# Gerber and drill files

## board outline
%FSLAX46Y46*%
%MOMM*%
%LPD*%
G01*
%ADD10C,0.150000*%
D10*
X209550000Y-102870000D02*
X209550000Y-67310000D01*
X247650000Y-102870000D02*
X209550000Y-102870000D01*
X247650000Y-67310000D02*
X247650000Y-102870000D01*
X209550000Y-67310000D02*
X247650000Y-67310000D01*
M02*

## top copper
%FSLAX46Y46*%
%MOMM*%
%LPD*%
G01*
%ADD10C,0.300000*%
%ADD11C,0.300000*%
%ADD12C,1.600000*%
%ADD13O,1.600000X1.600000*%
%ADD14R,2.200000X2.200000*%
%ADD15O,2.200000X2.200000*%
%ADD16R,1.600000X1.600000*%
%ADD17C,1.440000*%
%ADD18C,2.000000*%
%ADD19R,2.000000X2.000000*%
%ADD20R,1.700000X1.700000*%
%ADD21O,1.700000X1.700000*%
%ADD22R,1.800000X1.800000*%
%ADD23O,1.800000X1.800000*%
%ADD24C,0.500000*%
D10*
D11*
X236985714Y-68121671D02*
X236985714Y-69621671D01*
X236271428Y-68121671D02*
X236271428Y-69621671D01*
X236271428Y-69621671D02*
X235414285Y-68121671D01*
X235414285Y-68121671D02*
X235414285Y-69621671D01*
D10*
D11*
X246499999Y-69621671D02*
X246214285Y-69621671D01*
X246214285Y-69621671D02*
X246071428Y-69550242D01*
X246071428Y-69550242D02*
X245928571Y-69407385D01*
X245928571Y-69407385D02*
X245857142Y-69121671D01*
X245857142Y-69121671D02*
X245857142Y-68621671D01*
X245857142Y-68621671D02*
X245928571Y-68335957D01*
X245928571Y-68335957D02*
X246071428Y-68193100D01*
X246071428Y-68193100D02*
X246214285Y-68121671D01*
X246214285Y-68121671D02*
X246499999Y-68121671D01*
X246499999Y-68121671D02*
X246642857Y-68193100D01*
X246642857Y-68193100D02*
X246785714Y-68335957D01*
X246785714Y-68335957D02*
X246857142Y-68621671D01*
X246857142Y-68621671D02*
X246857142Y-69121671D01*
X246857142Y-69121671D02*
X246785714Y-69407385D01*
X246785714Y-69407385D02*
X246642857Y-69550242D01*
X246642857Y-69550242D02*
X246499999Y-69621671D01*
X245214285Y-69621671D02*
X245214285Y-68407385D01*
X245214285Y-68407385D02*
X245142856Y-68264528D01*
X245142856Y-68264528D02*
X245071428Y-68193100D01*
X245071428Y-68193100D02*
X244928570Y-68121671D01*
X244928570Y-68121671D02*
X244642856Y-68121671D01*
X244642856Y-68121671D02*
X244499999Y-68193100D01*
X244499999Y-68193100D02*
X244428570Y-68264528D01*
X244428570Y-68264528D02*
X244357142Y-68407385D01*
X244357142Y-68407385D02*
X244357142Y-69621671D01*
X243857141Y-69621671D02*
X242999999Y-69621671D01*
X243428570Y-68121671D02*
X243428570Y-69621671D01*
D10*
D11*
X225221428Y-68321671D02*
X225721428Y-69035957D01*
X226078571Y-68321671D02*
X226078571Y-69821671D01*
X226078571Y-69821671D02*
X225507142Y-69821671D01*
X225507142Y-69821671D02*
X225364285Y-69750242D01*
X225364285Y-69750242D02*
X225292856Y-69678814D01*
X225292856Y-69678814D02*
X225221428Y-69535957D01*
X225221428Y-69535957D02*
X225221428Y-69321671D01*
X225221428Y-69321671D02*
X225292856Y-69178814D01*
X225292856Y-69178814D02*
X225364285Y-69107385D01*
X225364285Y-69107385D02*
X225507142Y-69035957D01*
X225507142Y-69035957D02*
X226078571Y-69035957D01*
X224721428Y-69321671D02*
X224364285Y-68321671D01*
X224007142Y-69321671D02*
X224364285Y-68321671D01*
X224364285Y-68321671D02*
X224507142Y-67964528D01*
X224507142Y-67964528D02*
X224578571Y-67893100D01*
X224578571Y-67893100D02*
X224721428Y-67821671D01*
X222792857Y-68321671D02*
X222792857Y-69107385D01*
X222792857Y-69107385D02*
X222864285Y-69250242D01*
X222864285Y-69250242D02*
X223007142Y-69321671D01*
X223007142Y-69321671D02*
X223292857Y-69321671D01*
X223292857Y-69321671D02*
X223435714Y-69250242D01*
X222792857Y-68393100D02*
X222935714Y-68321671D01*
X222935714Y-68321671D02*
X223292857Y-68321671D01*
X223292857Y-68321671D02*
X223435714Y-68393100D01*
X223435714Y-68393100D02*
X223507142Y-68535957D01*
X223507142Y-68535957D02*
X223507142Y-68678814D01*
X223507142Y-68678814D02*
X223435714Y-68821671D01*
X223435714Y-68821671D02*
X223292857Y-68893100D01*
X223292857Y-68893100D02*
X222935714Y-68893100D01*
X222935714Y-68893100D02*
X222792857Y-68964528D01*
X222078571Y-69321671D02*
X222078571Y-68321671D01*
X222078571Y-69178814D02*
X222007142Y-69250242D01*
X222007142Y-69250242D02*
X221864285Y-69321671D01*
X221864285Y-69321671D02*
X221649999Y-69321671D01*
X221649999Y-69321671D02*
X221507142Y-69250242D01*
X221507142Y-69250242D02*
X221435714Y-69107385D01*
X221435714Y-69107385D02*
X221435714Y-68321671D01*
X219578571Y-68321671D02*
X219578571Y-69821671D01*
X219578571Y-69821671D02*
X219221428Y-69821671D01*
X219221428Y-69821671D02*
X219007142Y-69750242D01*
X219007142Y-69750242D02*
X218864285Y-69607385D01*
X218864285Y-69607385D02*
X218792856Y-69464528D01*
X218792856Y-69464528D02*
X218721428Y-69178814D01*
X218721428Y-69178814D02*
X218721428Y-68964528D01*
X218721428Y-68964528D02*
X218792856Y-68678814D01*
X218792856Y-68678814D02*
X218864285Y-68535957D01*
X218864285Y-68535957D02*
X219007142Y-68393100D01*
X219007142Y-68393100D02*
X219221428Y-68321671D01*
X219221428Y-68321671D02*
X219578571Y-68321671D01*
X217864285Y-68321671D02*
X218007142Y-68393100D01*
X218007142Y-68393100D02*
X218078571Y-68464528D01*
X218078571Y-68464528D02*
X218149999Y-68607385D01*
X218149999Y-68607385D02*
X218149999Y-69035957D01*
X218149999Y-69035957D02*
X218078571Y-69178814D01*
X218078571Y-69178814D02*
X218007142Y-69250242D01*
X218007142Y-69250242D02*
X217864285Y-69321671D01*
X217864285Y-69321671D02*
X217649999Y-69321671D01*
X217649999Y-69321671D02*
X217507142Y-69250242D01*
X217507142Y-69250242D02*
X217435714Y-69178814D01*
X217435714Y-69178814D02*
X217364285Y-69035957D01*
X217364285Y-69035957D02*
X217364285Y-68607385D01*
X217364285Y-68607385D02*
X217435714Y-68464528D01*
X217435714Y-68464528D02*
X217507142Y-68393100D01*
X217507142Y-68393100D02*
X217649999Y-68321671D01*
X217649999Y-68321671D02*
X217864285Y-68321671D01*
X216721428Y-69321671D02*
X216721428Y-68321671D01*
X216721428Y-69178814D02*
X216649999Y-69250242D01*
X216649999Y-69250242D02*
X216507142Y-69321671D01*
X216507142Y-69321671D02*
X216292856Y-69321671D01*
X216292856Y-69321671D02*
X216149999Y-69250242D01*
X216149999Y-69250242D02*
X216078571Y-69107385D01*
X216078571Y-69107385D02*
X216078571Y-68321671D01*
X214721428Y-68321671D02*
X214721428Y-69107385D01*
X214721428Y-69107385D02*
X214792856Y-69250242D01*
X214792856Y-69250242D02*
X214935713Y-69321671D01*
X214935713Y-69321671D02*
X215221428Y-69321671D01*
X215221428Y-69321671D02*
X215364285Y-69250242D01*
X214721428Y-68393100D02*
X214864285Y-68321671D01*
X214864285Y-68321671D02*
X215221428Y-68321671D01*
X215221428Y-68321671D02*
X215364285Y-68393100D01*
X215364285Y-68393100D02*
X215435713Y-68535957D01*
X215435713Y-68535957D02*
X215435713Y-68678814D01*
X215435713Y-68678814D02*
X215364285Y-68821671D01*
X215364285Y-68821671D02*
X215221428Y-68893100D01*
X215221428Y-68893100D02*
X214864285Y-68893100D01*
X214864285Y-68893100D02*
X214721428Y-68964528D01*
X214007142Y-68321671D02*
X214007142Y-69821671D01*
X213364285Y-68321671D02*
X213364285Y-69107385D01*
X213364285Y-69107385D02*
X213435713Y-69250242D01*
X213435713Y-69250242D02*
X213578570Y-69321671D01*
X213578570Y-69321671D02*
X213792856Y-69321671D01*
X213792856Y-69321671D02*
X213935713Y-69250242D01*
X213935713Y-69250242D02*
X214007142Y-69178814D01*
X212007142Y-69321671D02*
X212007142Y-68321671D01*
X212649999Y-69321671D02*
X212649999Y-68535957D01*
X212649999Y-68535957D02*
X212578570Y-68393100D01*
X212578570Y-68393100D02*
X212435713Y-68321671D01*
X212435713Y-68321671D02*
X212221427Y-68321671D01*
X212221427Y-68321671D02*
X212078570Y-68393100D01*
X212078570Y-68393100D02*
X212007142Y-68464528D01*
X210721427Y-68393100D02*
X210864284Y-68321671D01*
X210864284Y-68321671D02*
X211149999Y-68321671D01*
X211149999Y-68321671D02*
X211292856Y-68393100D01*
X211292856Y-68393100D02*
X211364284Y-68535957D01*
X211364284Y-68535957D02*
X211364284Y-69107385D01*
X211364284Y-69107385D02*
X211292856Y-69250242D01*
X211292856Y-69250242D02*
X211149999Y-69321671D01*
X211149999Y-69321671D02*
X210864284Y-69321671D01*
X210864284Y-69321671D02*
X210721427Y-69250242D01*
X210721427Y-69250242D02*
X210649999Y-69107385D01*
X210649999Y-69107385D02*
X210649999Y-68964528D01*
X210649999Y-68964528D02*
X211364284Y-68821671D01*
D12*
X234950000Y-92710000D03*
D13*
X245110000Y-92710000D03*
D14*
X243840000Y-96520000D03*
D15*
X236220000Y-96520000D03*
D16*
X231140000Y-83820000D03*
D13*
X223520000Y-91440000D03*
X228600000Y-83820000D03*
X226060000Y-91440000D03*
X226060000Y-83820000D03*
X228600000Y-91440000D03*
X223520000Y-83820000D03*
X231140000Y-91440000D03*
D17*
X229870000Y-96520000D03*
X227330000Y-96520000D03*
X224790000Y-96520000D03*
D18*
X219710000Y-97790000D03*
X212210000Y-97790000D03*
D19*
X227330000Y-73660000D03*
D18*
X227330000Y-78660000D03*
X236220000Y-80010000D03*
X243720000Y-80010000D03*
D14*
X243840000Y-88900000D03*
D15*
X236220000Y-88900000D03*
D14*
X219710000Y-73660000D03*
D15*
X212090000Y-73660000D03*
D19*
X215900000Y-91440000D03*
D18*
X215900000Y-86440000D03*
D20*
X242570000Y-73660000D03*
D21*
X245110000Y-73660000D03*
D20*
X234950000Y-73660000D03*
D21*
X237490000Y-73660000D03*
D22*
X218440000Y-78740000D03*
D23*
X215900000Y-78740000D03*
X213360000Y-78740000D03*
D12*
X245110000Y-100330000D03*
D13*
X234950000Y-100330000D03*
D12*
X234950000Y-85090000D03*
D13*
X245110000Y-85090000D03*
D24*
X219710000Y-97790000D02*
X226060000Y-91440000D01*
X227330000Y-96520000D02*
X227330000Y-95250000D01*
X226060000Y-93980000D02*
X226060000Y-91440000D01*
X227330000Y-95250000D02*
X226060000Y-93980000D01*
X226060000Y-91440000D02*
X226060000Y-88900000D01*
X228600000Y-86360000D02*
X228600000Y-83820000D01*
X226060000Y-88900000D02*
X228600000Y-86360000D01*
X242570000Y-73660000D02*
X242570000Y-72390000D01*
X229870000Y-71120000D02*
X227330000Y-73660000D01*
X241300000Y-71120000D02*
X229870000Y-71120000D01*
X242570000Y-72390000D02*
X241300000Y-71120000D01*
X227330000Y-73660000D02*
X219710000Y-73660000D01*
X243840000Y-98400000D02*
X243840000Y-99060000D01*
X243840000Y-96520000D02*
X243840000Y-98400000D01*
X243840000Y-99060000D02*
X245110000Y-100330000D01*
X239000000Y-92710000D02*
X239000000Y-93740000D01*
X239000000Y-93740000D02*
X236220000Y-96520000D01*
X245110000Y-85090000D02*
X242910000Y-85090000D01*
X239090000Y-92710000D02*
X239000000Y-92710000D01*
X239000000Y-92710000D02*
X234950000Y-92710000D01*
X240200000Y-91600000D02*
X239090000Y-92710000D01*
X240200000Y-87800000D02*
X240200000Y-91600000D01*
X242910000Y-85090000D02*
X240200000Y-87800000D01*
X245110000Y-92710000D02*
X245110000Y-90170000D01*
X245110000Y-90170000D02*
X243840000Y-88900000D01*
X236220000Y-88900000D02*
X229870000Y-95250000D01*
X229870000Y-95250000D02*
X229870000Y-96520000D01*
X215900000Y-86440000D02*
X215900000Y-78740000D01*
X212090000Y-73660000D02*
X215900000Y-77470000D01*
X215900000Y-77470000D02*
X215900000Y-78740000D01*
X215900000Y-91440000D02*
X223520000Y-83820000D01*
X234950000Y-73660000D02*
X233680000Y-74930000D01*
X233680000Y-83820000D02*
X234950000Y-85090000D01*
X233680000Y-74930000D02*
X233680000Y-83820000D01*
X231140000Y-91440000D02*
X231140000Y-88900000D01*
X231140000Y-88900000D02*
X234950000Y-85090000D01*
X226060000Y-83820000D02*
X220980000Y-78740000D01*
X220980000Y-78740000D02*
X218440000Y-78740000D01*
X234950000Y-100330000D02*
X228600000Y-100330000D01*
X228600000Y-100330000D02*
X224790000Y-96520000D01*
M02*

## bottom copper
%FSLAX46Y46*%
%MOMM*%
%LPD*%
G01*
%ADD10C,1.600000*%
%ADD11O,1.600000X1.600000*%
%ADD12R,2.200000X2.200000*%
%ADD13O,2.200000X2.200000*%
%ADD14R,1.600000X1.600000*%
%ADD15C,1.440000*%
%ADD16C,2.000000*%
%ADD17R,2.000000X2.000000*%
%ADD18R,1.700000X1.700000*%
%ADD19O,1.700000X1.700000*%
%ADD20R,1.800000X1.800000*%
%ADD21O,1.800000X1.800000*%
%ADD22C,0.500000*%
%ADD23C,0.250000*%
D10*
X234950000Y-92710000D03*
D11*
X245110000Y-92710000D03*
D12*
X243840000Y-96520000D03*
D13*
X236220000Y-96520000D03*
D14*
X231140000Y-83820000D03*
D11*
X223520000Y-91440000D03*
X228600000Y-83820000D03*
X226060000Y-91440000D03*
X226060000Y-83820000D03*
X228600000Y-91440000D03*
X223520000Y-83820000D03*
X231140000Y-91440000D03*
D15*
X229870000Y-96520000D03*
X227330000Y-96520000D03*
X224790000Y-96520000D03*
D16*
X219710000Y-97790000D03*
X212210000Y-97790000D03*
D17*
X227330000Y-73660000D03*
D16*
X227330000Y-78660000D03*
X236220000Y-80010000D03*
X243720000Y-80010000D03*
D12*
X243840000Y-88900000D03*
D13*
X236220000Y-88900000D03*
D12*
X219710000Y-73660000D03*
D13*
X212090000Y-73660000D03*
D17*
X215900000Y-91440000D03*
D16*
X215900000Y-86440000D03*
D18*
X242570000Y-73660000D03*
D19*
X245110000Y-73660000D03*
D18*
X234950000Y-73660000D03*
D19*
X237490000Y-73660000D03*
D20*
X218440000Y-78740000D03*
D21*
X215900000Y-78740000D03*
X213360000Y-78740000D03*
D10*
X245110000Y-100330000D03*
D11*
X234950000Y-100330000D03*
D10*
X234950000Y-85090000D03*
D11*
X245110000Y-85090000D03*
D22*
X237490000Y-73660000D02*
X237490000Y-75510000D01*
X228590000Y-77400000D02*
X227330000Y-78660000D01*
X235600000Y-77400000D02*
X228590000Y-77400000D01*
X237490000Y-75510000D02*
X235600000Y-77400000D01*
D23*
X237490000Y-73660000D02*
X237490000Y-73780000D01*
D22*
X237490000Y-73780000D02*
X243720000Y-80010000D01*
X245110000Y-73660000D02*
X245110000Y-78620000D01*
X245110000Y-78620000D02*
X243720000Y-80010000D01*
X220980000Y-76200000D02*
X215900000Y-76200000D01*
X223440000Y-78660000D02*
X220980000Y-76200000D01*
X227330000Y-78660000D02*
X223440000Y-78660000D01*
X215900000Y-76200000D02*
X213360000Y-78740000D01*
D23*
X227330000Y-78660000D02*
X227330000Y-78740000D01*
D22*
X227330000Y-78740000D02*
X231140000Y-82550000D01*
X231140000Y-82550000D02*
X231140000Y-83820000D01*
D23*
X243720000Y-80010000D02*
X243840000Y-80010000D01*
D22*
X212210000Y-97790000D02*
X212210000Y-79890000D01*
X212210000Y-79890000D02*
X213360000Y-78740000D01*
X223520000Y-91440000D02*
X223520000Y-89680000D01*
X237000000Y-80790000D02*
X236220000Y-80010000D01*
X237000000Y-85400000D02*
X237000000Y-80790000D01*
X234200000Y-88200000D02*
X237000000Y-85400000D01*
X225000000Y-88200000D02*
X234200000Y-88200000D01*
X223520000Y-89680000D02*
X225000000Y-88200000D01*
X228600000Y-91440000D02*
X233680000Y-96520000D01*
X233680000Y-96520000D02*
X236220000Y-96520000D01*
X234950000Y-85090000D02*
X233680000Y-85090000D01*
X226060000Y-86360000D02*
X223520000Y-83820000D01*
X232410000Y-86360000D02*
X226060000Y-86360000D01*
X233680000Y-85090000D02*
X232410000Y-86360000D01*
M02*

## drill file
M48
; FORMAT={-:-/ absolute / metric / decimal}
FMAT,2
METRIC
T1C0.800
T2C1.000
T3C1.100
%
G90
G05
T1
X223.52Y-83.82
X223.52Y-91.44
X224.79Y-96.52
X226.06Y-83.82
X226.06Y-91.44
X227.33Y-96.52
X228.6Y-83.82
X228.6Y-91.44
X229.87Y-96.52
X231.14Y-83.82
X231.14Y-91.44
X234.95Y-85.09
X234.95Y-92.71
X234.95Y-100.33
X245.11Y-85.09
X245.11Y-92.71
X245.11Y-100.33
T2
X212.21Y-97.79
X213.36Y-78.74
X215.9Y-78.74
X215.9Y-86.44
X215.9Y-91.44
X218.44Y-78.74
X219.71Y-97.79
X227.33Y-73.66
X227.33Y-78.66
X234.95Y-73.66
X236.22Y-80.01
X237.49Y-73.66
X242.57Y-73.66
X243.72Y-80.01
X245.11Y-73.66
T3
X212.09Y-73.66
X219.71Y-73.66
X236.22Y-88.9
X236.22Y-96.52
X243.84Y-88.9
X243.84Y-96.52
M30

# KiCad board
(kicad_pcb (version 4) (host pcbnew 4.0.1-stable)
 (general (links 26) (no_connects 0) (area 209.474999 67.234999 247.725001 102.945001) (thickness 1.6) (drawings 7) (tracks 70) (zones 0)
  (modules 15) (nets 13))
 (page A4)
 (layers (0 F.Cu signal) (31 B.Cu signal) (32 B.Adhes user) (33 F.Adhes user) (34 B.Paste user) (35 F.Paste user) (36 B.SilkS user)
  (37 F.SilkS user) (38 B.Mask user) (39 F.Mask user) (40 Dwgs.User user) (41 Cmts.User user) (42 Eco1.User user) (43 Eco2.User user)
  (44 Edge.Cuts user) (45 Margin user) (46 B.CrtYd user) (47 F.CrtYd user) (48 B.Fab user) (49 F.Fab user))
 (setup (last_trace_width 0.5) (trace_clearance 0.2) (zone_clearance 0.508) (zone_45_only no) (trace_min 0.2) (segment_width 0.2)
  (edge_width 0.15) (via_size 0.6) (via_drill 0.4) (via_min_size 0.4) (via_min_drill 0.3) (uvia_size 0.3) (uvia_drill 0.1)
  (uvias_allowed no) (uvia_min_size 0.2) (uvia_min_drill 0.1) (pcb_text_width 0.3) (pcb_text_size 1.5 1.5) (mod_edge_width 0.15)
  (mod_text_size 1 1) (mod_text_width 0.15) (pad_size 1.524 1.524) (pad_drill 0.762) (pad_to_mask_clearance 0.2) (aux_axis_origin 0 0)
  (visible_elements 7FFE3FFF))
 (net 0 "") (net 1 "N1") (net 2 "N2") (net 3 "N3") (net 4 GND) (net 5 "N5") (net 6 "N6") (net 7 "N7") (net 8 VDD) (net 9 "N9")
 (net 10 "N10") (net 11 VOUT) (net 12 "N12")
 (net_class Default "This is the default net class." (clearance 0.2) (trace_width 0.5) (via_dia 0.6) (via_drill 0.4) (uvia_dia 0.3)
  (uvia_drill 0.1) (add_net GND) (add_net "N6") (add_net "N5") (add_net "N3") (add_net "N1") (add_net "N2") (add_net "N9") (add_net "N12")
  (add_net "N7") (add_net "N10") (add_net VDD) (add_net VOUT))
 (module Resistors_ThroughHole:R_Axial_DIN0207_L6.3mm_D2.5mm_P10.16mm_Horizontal (layer F.Cu) (at 234.95 92.71)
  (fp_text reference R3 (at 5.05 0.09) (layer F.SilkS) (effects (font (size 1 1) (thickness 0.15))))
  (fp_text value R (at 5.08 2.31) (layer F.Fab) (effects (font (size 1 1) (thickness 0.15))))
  (pad 1 thru_hole circle (at 0 0) (size 1.6 1.6) (drill 0.8) (layers *.Cu *.Mask) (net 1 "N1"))
  (pad 2 thru_hole oval (at 10.16 0) (size 1.6 1.6) (drill 0.8) (layers *.Cu *.Mask) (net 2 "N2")))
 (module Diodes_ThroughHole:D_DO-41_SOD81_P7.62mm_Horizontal (layer F.Cu) (at 243.84 96.52 180)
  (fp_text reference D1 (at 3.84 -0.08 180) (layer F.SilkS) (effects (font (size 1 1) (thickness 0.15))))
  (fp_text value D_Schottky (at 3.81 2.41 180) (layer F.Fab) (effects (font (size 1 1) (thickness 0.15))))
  (pad 1 thru_hole rect (at 0 0 180) (size 2.2 2.2) (drill 1.1) (layers *.Cu *.Mask) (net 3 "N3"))
  (pad 2 thru_hole oval (at 7.62 0 180) (size 2.2 2.2) (drill 1.1) (layers *.Cu *.Mask) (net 1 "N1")))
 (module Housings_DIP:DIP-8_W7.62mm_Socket (layer F.Cu) (at 231.14 83.82 270)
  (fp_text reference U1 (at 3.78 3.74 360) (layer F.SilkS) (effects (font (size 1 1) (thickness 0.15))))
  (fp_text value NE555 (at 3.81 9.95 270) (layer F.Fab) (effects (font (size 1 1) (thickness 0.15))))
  (pad 1 thru_hole rect (at 0 0 270) (size 1.6 1.6) (drill 0.8) (layers *.Cu *.Mask) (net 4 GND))
  (pad 5 thru_hole oval (at 7.62 7.62 270) (size 1.6 1.6) (drill 0.8) (layers *.Cu *.Mask) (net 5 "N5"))
  (pad 2 thru_hole oval (at 0 2.54 270) (size 1.6 1.6) (drill 0.8) (layers *.Cu *.Mask) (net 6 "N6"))
  (pad 6 thru_hole oval (at 7.62 5.08 270) (size 1.6 1.6) (drill 0.8) (layers *.Cu *.Mask) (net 6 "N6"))
  (pad 3 thru_hole oval (at 0 5.08 270) (size 1.6 1.6) (drill 0.8) (layers *.Cu *.Mask) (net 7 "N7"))
  (pad 7 thru_hole oval (at 7.62 2.54 270) (size 1.6 1.6) (drill 0.8) (layers *.Cu *.Mask) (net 1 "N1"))
  (pad 4 thru_hole oval (at 0 7.62 270) (size 1.6 1.6) (drill 0.8) (layers *.Cu *.Mask) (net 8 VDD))
  (pad 8 thru_hole oval (at 7.62 0 270) (size 1.6 1.6) (drill 0.8) (layers *.Cu *.Mask) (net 8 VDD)))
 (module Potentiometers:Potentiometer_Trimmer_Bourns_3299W (layer F.Cu) (at 229.87 96.52)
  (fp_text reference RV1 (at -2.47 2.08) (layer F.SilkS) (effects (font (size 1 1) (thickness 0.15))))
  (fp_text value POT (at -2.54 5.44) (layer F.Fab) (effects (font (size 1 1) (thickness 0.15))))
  (pad 1 thru_hole circle (at 0 0) (size 1.44 1.44) (drill 0.8) (layers *.Cu *.Mask) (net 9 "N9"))
  (pad 2 thru_hole circle (at -2.54 0) (size 1.44 1.44) (drill 0.8) (layers *.Cu *.Mask) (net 6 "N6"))
  (pad 3 thru_hole circle (at -5.08 0) (size 1.44 1.44) (drill 0.8) (layers *.Cu *.Mask) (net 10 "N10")))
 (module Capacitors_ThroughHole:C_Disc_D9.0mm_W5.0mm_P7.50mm (layer F.Cu) (at 219.71 97.79 180)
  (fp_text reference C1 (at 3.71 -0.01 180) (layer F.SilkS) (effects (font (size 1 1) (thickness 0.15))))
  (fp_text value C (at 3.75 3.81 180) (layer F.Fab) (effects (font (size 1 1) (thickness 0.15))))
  (pad 1 thru_hole circle (at 0 0 180) (size 2 2) (drill 1) (layers *.Cu *.Mask) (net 6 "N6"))
  (pad 2 thru_hole circle (at 7.5 0 180) (size 2 2) (drill 1) (layers *.Cu *.Mask) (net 4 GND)))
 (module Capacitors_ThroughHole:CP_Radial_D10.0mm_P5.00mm (layer F.Cu) (at 227.33 73.66 270)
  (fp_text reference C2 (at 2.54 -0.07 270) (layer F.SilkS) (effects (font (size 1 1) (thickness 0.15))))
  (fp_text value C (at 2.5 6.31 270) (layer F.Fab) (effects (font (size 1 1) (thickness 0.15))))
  (pad 1 thru_hole rect (at 0 0 270) (size 2 2) (drill 1) (layers *.Cu *.Mask) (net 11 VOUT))
  (pad 2 thru_hole circle (at 5 0 270) (size 2 2) (drill 1) (layers *.Cu *.Mask) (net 4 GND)))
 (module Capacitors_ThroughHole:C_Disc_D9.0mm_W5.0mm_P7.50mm (layer F.Cu) (at 236.22 80.01)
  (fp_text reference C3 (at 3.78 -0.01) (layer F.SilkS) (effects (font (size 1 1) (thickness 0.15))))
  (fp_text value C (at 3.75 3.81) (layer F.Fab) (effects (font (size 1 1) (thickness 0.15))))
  (pad 1 thru_hole circle (at 0 0) (size 2 2) (drill 1) (layers *.Cu *.Mask) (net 5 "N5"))
  (pad 2 thru_hole circle (at 7.5 0) (size 2 2) (drill 1) (layers *.Cu *.Mask) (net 4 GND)))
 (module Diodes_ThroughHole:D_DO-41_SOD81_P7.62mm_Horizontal (layer F.Cu) (at 243.84 88.9 180)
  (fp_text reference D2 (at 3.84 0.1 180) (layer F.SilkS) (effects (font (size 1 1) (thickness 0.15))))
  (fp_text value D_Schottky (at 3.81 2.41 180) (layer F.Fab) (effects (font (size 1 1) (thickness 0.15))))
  (pad 1 thru_hole rect (at 0 0 180) (size 2.2 2.2) (drill 1.1) (layers *.Cu *.Mask) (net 2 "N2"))
  (pad 2 thru_hole oval (at 7.62 0 180) (size 2.2 2.2) (drill 1.1) (layers *.Cu *.Mask) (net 9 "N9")))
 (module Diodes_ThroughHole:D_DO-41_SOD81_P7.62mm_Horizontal (layer F.Cu) (at 219.71 73.66 180)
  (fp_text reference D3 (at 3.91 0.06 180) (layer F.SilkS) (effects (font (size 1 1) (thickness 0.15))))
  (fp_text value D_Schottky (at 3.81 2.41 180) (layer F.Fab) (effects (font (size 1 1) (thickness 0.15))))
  (pad 1 thru_hole rect (at 0 0 180) (size 2.2 2.2) (drill 1.1) (layers *.Cu *.Mask) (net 11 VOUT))
  (pad 2 thru_hole oval (at 7.62 0 180) (size 2.2 2.2) (drill 1.1) (layers *.Cu *.Mask) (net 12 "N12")))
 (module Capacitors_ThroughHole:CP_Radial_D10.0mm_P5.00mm (layer F.Cu) (at 215.9 91.44 90)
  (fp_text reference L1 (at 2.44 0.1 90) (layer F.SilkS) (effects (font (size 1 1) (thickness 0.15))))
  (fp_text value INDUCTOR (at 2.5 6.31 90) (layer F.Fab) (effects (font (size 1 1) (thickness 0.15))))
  (pad 1 thru_hole rect (at 0 0 90) (size 2 2) (drill 1) (layers *.Cu *.Mask) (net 8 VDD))
  (pad 2 thru_hole circle (at 5 0 90) (size 2 2) (drill 1) (layers *.Cu *.Mask) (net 12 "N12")))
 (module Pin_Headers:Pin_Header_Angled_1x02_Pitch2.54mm (layer F.Cu) (at 242.57 73.66 90)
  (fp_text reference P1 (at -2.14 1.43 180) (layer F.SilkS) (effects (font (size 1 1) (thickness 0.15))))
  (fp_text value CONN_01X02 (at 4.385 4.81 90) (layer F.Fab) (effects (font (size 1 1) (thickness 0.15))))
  (pad 1 thru_hole rect (at 0 0 90) (size 1.7 1.7) (drill 1) (layers *.Cu *.Mask) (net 11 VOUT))
  (pad 2 thru_hole oval (at 0 2.54 90) (size 1.7 1.7) (drill 1) (layers *.Cu *.Mask) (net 4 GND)))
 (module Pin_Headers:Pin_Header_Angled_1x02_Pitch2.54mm (layer F.Cu) (at 234.95 73.66 90)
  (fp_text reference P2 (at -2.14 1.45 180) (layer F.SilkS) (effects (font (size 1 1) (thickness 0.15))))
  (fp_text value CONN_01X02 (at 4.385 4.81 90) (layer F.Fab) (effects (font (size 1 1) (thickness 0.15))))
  (pad 1 thru_hole rect (at 0 0 90) (size 1.7 1.7) (drill 1) (layers *.Cu *.Mask) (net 8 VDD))
  (pad 2 thru_hole oval (at 0 2.54 90) (size 1.7 1.7) (drill 1) (layers *.Cu *.Mask) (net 4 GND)))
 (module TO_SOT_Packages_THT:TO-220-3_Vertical (layer F.Cu) (at 218.44 78.74 180)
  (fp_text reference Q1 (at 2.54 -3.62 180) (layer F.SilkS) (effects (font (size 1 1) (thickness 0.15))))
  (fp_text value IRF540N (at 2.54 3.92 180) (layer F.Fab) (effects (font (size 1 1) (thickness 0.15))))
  (pad 1 thru_hole rect (at 0 0 180) (size 1.8 1.8) (drill 1) (layers *.Cu *.Mask) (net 7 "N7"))
  (pad 2 thru_hole oval (at 2.54 0 180) (size 1.8 1.8) (drill 1) (layers *.Cu *.Mask) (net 12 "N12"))
  (pad 3 thru_hole oval (at 5.08 0 180) (size 1.8 1.8) (drill 1) (layers *.Cu *.Mask) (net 4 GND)))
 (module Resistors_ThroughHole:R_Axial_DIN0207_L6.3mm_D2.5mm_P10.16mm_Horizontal (layer F.Cu) (at 245.11 100.33 180)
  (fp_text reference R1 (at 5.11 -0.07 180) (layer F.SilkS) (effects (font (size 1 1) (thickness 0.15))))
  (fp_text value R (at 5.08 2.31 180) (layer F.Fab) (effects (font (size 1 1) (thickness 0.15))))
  (pad 1 thru_hole circle (at 0 0 180) (size 1.6 1.6) (drill 0.8) (layers *.Cu *.Mask) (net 3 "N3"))
  (pad 2 thru_hole oval (at 10.16 0 180) (size 1.6 1.6) (drill 0.8) (layers *.Cu *.Mask) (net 10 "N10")))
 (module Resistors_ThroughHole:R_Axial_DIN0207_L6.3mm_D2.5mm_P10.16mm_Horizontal (layer F.Cu) (at 234.95 85.09)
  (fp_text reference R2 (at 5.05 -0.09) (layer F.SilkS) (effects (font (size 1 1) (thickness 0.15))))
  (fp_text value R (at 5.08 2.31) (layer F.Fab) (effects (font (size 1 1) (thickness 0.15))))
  (pad 1 thru_hole circle (at 0 0) (size 1.6 1.6) (drill 0.8) (layers *.Cu *.Mask) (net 8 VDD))
  (pad 2 thru_hole oval (at 10.16 0) (size 1.6 1.6) (drill 0.8) (layers *.Cu *.Mask) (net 1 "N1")))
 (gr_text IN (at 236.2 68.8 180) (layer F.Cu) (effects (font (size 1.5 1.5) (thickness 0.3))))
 (gr_line (start 209.55 102.87) (end 209.55 67.31) (angle 90) (layer Edge.Cuts) (width 0.15))
 (gr_line (start 247.65 102.87) (end 209.55 102.87) (angle 90) (layer Edge.Cuts) (width 0.15))
 (gr_line (start 247.65 67.31) (end 247.65 102.87) (angle 90) (layer Edge.Cuts) (width 0.15))
 (gr_line (start 209.55 67.31) (end 247.65 67.31) (angle 90) (layer Edge.Cuts) (width 0.15))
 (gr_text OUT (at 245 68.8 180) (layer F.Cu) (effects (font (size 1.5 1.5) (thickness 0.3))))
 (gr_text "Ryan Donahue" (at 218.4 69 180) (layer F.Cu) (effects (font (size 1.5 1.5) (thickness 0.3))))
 (segment (start 219.71 97.79) (end 226.06 91.44) (width 0.5) (layer F.Cu) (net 6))
 (segment (start 227.33 96.52) (end 227.33 95.25) (width 0.5) (layer F.Cu) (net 6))
 (segment (start 226.06 93.98) (end 226.06 91.44) (width 0.5) (layer F.Cu) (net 6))
 (segment (start 227.33 95.25) (end 226.06 93.98) (width 0.5) (layer F.Cu) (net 6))
 (segment (start 226.06 91.44) (end 226.06 88.9) (width 0.5) (layer F.Cu) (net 6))
 (segment (start 228.6 86.36) (end 228.6 83.82) (width 0.5) (layer F.Cu) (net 6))
 (segment (start 226.06 88.9) (end 228.6 86.36) (width 0.5) (layer F.Cu) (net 6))
 (segment (start 237.49 73.66) (end 237.49 75.51) (width 0.5) (layer B.Cu) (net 4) (status 400000))
 (segment (start 228.59 77.4) (end 227.33 78.66) (width 0.5) (layer B.Cu) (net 4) (status 800000))
 (segment (start 235.6 77.4) (end 228.59 77.4) (width 0.5) (layer B.Cu) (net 4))
 (segment (start 237.49 75.51) (end 235.6 77.4) (width 0.5) (layer B.Cu) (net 4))
 (segment (start 237.49 73.66) (end 237.49 73.78) (width 0.25) (layer B.Cu) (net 4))
 (segment (start 237.49 73.78) (end 243.72 80.01) (width 0.5) (layer B.Cu) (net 4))
 (segment (start 245.11 73.66) (end 245.11 78.62) (width 0.5) (layer B.Cu) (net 4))
 (segment (start 245.11 78.62) (end 243.72 80.01) (width 0.5) (layer B.Cu) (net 4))
 (segment (start 220.98 76.2) (end 215.9 76.2) (width 0.5) (layer B.Cu) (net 4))
 (segment (start 223.44 78.66) (end 220.98 76.2) (width 0.5) (layer B.Cu) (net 4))
 (segment (start 227.33 78.66) (end 223.44 78.66) (width 0.5) (layer B.Cu) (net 4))
 (segment (start 215.9 76.2) (end 213.36 78.74) (width 0.5) (layer B.Cu) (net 4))
 (segment (start 227.33 78.66) (end 227.33 78.74) (width 0.25) (layer B.Cu) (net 4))
 (segment (start 227.33 78.74) (end 231.14 82.55) (width 0.5) (layer B.Cu) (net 4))
 (segment (start 231.14 82.55) (end 231.14 83.82) (width 0.5) (layer B.Cu) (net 4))
 (segment (start 243.72 80.01) (end 243.84 80.01) (width 0.25) (layer B.Cu) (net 4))
 (segment (start 212.21 97.79) (end 212.21 79.89) (width 0.5) (layer B.Cu) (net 4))
 (segment (start 212.21 79.89) (end 213.36 78.74) (width 0.5) (layer B.Cu) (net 4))
 (segment (start 242.57 73.66) (end 242.57 72.39) (width 0.5) (layer F.Cu) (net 11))
 (segment (start 229.87 71.12) (end 227.33 73.66) (width 0.5) (layer F.Cu) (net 11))
 (segment (start 241.3 71.12) (end 229.87 71.12) (width 0.5) (layer F.Cu) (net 11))
 (segment (start 242.57 72.39) (end 241.3 71.12) (width 0.5) (layer F.Cu) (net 11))
 (segment (start 227.33 73.66) (end 219.71 73.66) (width 0.5) (layer F.Cu) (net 11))
 (segment (start 223.52 91.44) (end 223.52 89.68) (width 0.5) (layer B.Cu) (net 5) (status 400000))
 (segment (start 237 80.79) (end 236.22 80.01) (width 0.5) (layer B.Cu) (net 5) (status 800000))
 (segment (start 237 85.4) (end 237 80.79) (width 0.5) (layer B.Cu) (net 5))
 (segment (start 234.2 88.2) (end 237 85.4) (width 0.5) (layer B.Cu) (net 5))
 (segment (start 225 88.2) (end 234.2 88.2) (width 0.5) (layer B.Cu) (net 5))
 (segment (start 223.52 89.68) (end 225 88.2) (width 0.5) (layer B.Cu) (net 5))
 (segment (start 243.84 98.4) (end 243.84 99.06) (width 0.5) (layer F.Cu) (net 3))
 (segment (start 243.84 96.52) (end 243.84 98.4) (width 0.5) (layer F.Cu) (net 3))
 (segment (start 243.84 99.06) (end 245.11 100.33) (width 0.5) (layer F.Cu) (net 3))
 (segment (start 239 92.71) (end 239 93.74) (width 0.5) (layer F.Cu) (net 1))
 (segment (start 239 93.74) (end 236.22 96.52) (width 0.5) (layer F.Cu) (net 1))
 (segment (start 245.11 85.09) (end 242.91 85.09) (width 0.5) (layer F.Cu) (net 1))
 (segment (start 239.09 92.71) (end 239 92.71) (width 0.5) (layer F.Cu) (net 1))
 (segment (start 239 92.71) (end 234.95 92.71) (width 0.5) (layer F.Cu) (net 1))
 (segment (start 240.2 91.6) (end 239.09 92.71) (width 0.5) (layer F.Cu) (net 1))
 (segment (start 240.2 87.8) (end 240.2 91.6) (width 0.5) (layer F.Cu) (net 1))
 (segment (start 242.91 85.09) (end 240.2 87.8) (width 0.5) (layer F.Cu) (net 1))
 (segment (start 228.6 91.44) (end 233.68 96.52) (width 0.5) (layer B.Cu) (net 1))
 (segment (start 233.68 96.52) (end 236.22 96.52) (width 0.5) (layer B.Cu) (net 1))
 (segment (start 245.11 92.71) (end 245.11 90.17) (width 0.5) (layer F.Cu) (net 2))
 (segment (start 245.11 90.17) (end 243.84 88.9) (width 0.5) (layer F.Cu) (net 2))
 (segment (start 236.22 88.9) (end 229.87 95.25) (width 0.5) (layer F.Cu) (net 9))
 (segment (start 229.87 95.25) (end 229.87 96.52) (width 0.5) (layer F.Cu) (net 9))
 (segment (start 215.9 86.44) (end 215.9 78.74) (width 0.5) (layer F.Cu) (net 12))
 (segment (start 212.09 73.66) (end 215.9 77.47) (width 0.5) (layer F.Cu) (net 12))
 (segment (start 215.9 77.47) (end 215.9 78.74) (width 0.5) (layer F.Cu) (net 12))
 (segment (start 234.95 85.09) (end 233.68 85.09) (width 0.5) (layer B.Cu) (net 8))
 (segment (start 226.06 86.36) (end 223.52 83.82) (width 0.5) (layer B.Cu) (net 8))
 (segment (start 232.41 86.36) (end 226.06 86.36) (width 0.5) (layer B.Cu) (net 8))
 (segment (start 233.68 85.09) (end 232.41 86.36) (width 0.5) (layer B.Cu) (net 8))
 (segment (start 215.9 91.44) (end 223.52 83.82) (width 0.5) (layer F.Cu) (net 8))
 (segment (start 234.95 73.66) (end 233.68 74.93) (width 0.5) (layer F.Cu) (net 8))
 (segment (start 233.68 83.82) (end 234.95 85.09) (width 0.5) (layer F.Cu) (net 8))
 (segment (start 233.68 74.93) (end 233.68 83.82) (width 0.5) (layer F.Cu) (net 8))
 (segment (start 231.14 91.44) (end 231.14 88.9) (width 0.5) (layer F.Cu) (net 8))
 (segment (start 231.14 88.9) (end 234.95 85.09) (width 0.5) (layer F.Cu) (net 8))
 (segment (start 226.06 83.82) (end 220.98 78.74) (width 0.5) (layer F.Cu) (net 7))
 (segment (start 220.98 78.74) (end 218.44 78.74) (width 0.5) (layer F.Cu) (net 7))
 (segment (start 234.95 100.33) (end 228.6 100.33) (width 0.5) (layer F.Cu) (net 10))
 (segment (start 228.6 100.33) (end 224.79 96.52) (width 0.5) (layer F.Cu) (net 10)))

